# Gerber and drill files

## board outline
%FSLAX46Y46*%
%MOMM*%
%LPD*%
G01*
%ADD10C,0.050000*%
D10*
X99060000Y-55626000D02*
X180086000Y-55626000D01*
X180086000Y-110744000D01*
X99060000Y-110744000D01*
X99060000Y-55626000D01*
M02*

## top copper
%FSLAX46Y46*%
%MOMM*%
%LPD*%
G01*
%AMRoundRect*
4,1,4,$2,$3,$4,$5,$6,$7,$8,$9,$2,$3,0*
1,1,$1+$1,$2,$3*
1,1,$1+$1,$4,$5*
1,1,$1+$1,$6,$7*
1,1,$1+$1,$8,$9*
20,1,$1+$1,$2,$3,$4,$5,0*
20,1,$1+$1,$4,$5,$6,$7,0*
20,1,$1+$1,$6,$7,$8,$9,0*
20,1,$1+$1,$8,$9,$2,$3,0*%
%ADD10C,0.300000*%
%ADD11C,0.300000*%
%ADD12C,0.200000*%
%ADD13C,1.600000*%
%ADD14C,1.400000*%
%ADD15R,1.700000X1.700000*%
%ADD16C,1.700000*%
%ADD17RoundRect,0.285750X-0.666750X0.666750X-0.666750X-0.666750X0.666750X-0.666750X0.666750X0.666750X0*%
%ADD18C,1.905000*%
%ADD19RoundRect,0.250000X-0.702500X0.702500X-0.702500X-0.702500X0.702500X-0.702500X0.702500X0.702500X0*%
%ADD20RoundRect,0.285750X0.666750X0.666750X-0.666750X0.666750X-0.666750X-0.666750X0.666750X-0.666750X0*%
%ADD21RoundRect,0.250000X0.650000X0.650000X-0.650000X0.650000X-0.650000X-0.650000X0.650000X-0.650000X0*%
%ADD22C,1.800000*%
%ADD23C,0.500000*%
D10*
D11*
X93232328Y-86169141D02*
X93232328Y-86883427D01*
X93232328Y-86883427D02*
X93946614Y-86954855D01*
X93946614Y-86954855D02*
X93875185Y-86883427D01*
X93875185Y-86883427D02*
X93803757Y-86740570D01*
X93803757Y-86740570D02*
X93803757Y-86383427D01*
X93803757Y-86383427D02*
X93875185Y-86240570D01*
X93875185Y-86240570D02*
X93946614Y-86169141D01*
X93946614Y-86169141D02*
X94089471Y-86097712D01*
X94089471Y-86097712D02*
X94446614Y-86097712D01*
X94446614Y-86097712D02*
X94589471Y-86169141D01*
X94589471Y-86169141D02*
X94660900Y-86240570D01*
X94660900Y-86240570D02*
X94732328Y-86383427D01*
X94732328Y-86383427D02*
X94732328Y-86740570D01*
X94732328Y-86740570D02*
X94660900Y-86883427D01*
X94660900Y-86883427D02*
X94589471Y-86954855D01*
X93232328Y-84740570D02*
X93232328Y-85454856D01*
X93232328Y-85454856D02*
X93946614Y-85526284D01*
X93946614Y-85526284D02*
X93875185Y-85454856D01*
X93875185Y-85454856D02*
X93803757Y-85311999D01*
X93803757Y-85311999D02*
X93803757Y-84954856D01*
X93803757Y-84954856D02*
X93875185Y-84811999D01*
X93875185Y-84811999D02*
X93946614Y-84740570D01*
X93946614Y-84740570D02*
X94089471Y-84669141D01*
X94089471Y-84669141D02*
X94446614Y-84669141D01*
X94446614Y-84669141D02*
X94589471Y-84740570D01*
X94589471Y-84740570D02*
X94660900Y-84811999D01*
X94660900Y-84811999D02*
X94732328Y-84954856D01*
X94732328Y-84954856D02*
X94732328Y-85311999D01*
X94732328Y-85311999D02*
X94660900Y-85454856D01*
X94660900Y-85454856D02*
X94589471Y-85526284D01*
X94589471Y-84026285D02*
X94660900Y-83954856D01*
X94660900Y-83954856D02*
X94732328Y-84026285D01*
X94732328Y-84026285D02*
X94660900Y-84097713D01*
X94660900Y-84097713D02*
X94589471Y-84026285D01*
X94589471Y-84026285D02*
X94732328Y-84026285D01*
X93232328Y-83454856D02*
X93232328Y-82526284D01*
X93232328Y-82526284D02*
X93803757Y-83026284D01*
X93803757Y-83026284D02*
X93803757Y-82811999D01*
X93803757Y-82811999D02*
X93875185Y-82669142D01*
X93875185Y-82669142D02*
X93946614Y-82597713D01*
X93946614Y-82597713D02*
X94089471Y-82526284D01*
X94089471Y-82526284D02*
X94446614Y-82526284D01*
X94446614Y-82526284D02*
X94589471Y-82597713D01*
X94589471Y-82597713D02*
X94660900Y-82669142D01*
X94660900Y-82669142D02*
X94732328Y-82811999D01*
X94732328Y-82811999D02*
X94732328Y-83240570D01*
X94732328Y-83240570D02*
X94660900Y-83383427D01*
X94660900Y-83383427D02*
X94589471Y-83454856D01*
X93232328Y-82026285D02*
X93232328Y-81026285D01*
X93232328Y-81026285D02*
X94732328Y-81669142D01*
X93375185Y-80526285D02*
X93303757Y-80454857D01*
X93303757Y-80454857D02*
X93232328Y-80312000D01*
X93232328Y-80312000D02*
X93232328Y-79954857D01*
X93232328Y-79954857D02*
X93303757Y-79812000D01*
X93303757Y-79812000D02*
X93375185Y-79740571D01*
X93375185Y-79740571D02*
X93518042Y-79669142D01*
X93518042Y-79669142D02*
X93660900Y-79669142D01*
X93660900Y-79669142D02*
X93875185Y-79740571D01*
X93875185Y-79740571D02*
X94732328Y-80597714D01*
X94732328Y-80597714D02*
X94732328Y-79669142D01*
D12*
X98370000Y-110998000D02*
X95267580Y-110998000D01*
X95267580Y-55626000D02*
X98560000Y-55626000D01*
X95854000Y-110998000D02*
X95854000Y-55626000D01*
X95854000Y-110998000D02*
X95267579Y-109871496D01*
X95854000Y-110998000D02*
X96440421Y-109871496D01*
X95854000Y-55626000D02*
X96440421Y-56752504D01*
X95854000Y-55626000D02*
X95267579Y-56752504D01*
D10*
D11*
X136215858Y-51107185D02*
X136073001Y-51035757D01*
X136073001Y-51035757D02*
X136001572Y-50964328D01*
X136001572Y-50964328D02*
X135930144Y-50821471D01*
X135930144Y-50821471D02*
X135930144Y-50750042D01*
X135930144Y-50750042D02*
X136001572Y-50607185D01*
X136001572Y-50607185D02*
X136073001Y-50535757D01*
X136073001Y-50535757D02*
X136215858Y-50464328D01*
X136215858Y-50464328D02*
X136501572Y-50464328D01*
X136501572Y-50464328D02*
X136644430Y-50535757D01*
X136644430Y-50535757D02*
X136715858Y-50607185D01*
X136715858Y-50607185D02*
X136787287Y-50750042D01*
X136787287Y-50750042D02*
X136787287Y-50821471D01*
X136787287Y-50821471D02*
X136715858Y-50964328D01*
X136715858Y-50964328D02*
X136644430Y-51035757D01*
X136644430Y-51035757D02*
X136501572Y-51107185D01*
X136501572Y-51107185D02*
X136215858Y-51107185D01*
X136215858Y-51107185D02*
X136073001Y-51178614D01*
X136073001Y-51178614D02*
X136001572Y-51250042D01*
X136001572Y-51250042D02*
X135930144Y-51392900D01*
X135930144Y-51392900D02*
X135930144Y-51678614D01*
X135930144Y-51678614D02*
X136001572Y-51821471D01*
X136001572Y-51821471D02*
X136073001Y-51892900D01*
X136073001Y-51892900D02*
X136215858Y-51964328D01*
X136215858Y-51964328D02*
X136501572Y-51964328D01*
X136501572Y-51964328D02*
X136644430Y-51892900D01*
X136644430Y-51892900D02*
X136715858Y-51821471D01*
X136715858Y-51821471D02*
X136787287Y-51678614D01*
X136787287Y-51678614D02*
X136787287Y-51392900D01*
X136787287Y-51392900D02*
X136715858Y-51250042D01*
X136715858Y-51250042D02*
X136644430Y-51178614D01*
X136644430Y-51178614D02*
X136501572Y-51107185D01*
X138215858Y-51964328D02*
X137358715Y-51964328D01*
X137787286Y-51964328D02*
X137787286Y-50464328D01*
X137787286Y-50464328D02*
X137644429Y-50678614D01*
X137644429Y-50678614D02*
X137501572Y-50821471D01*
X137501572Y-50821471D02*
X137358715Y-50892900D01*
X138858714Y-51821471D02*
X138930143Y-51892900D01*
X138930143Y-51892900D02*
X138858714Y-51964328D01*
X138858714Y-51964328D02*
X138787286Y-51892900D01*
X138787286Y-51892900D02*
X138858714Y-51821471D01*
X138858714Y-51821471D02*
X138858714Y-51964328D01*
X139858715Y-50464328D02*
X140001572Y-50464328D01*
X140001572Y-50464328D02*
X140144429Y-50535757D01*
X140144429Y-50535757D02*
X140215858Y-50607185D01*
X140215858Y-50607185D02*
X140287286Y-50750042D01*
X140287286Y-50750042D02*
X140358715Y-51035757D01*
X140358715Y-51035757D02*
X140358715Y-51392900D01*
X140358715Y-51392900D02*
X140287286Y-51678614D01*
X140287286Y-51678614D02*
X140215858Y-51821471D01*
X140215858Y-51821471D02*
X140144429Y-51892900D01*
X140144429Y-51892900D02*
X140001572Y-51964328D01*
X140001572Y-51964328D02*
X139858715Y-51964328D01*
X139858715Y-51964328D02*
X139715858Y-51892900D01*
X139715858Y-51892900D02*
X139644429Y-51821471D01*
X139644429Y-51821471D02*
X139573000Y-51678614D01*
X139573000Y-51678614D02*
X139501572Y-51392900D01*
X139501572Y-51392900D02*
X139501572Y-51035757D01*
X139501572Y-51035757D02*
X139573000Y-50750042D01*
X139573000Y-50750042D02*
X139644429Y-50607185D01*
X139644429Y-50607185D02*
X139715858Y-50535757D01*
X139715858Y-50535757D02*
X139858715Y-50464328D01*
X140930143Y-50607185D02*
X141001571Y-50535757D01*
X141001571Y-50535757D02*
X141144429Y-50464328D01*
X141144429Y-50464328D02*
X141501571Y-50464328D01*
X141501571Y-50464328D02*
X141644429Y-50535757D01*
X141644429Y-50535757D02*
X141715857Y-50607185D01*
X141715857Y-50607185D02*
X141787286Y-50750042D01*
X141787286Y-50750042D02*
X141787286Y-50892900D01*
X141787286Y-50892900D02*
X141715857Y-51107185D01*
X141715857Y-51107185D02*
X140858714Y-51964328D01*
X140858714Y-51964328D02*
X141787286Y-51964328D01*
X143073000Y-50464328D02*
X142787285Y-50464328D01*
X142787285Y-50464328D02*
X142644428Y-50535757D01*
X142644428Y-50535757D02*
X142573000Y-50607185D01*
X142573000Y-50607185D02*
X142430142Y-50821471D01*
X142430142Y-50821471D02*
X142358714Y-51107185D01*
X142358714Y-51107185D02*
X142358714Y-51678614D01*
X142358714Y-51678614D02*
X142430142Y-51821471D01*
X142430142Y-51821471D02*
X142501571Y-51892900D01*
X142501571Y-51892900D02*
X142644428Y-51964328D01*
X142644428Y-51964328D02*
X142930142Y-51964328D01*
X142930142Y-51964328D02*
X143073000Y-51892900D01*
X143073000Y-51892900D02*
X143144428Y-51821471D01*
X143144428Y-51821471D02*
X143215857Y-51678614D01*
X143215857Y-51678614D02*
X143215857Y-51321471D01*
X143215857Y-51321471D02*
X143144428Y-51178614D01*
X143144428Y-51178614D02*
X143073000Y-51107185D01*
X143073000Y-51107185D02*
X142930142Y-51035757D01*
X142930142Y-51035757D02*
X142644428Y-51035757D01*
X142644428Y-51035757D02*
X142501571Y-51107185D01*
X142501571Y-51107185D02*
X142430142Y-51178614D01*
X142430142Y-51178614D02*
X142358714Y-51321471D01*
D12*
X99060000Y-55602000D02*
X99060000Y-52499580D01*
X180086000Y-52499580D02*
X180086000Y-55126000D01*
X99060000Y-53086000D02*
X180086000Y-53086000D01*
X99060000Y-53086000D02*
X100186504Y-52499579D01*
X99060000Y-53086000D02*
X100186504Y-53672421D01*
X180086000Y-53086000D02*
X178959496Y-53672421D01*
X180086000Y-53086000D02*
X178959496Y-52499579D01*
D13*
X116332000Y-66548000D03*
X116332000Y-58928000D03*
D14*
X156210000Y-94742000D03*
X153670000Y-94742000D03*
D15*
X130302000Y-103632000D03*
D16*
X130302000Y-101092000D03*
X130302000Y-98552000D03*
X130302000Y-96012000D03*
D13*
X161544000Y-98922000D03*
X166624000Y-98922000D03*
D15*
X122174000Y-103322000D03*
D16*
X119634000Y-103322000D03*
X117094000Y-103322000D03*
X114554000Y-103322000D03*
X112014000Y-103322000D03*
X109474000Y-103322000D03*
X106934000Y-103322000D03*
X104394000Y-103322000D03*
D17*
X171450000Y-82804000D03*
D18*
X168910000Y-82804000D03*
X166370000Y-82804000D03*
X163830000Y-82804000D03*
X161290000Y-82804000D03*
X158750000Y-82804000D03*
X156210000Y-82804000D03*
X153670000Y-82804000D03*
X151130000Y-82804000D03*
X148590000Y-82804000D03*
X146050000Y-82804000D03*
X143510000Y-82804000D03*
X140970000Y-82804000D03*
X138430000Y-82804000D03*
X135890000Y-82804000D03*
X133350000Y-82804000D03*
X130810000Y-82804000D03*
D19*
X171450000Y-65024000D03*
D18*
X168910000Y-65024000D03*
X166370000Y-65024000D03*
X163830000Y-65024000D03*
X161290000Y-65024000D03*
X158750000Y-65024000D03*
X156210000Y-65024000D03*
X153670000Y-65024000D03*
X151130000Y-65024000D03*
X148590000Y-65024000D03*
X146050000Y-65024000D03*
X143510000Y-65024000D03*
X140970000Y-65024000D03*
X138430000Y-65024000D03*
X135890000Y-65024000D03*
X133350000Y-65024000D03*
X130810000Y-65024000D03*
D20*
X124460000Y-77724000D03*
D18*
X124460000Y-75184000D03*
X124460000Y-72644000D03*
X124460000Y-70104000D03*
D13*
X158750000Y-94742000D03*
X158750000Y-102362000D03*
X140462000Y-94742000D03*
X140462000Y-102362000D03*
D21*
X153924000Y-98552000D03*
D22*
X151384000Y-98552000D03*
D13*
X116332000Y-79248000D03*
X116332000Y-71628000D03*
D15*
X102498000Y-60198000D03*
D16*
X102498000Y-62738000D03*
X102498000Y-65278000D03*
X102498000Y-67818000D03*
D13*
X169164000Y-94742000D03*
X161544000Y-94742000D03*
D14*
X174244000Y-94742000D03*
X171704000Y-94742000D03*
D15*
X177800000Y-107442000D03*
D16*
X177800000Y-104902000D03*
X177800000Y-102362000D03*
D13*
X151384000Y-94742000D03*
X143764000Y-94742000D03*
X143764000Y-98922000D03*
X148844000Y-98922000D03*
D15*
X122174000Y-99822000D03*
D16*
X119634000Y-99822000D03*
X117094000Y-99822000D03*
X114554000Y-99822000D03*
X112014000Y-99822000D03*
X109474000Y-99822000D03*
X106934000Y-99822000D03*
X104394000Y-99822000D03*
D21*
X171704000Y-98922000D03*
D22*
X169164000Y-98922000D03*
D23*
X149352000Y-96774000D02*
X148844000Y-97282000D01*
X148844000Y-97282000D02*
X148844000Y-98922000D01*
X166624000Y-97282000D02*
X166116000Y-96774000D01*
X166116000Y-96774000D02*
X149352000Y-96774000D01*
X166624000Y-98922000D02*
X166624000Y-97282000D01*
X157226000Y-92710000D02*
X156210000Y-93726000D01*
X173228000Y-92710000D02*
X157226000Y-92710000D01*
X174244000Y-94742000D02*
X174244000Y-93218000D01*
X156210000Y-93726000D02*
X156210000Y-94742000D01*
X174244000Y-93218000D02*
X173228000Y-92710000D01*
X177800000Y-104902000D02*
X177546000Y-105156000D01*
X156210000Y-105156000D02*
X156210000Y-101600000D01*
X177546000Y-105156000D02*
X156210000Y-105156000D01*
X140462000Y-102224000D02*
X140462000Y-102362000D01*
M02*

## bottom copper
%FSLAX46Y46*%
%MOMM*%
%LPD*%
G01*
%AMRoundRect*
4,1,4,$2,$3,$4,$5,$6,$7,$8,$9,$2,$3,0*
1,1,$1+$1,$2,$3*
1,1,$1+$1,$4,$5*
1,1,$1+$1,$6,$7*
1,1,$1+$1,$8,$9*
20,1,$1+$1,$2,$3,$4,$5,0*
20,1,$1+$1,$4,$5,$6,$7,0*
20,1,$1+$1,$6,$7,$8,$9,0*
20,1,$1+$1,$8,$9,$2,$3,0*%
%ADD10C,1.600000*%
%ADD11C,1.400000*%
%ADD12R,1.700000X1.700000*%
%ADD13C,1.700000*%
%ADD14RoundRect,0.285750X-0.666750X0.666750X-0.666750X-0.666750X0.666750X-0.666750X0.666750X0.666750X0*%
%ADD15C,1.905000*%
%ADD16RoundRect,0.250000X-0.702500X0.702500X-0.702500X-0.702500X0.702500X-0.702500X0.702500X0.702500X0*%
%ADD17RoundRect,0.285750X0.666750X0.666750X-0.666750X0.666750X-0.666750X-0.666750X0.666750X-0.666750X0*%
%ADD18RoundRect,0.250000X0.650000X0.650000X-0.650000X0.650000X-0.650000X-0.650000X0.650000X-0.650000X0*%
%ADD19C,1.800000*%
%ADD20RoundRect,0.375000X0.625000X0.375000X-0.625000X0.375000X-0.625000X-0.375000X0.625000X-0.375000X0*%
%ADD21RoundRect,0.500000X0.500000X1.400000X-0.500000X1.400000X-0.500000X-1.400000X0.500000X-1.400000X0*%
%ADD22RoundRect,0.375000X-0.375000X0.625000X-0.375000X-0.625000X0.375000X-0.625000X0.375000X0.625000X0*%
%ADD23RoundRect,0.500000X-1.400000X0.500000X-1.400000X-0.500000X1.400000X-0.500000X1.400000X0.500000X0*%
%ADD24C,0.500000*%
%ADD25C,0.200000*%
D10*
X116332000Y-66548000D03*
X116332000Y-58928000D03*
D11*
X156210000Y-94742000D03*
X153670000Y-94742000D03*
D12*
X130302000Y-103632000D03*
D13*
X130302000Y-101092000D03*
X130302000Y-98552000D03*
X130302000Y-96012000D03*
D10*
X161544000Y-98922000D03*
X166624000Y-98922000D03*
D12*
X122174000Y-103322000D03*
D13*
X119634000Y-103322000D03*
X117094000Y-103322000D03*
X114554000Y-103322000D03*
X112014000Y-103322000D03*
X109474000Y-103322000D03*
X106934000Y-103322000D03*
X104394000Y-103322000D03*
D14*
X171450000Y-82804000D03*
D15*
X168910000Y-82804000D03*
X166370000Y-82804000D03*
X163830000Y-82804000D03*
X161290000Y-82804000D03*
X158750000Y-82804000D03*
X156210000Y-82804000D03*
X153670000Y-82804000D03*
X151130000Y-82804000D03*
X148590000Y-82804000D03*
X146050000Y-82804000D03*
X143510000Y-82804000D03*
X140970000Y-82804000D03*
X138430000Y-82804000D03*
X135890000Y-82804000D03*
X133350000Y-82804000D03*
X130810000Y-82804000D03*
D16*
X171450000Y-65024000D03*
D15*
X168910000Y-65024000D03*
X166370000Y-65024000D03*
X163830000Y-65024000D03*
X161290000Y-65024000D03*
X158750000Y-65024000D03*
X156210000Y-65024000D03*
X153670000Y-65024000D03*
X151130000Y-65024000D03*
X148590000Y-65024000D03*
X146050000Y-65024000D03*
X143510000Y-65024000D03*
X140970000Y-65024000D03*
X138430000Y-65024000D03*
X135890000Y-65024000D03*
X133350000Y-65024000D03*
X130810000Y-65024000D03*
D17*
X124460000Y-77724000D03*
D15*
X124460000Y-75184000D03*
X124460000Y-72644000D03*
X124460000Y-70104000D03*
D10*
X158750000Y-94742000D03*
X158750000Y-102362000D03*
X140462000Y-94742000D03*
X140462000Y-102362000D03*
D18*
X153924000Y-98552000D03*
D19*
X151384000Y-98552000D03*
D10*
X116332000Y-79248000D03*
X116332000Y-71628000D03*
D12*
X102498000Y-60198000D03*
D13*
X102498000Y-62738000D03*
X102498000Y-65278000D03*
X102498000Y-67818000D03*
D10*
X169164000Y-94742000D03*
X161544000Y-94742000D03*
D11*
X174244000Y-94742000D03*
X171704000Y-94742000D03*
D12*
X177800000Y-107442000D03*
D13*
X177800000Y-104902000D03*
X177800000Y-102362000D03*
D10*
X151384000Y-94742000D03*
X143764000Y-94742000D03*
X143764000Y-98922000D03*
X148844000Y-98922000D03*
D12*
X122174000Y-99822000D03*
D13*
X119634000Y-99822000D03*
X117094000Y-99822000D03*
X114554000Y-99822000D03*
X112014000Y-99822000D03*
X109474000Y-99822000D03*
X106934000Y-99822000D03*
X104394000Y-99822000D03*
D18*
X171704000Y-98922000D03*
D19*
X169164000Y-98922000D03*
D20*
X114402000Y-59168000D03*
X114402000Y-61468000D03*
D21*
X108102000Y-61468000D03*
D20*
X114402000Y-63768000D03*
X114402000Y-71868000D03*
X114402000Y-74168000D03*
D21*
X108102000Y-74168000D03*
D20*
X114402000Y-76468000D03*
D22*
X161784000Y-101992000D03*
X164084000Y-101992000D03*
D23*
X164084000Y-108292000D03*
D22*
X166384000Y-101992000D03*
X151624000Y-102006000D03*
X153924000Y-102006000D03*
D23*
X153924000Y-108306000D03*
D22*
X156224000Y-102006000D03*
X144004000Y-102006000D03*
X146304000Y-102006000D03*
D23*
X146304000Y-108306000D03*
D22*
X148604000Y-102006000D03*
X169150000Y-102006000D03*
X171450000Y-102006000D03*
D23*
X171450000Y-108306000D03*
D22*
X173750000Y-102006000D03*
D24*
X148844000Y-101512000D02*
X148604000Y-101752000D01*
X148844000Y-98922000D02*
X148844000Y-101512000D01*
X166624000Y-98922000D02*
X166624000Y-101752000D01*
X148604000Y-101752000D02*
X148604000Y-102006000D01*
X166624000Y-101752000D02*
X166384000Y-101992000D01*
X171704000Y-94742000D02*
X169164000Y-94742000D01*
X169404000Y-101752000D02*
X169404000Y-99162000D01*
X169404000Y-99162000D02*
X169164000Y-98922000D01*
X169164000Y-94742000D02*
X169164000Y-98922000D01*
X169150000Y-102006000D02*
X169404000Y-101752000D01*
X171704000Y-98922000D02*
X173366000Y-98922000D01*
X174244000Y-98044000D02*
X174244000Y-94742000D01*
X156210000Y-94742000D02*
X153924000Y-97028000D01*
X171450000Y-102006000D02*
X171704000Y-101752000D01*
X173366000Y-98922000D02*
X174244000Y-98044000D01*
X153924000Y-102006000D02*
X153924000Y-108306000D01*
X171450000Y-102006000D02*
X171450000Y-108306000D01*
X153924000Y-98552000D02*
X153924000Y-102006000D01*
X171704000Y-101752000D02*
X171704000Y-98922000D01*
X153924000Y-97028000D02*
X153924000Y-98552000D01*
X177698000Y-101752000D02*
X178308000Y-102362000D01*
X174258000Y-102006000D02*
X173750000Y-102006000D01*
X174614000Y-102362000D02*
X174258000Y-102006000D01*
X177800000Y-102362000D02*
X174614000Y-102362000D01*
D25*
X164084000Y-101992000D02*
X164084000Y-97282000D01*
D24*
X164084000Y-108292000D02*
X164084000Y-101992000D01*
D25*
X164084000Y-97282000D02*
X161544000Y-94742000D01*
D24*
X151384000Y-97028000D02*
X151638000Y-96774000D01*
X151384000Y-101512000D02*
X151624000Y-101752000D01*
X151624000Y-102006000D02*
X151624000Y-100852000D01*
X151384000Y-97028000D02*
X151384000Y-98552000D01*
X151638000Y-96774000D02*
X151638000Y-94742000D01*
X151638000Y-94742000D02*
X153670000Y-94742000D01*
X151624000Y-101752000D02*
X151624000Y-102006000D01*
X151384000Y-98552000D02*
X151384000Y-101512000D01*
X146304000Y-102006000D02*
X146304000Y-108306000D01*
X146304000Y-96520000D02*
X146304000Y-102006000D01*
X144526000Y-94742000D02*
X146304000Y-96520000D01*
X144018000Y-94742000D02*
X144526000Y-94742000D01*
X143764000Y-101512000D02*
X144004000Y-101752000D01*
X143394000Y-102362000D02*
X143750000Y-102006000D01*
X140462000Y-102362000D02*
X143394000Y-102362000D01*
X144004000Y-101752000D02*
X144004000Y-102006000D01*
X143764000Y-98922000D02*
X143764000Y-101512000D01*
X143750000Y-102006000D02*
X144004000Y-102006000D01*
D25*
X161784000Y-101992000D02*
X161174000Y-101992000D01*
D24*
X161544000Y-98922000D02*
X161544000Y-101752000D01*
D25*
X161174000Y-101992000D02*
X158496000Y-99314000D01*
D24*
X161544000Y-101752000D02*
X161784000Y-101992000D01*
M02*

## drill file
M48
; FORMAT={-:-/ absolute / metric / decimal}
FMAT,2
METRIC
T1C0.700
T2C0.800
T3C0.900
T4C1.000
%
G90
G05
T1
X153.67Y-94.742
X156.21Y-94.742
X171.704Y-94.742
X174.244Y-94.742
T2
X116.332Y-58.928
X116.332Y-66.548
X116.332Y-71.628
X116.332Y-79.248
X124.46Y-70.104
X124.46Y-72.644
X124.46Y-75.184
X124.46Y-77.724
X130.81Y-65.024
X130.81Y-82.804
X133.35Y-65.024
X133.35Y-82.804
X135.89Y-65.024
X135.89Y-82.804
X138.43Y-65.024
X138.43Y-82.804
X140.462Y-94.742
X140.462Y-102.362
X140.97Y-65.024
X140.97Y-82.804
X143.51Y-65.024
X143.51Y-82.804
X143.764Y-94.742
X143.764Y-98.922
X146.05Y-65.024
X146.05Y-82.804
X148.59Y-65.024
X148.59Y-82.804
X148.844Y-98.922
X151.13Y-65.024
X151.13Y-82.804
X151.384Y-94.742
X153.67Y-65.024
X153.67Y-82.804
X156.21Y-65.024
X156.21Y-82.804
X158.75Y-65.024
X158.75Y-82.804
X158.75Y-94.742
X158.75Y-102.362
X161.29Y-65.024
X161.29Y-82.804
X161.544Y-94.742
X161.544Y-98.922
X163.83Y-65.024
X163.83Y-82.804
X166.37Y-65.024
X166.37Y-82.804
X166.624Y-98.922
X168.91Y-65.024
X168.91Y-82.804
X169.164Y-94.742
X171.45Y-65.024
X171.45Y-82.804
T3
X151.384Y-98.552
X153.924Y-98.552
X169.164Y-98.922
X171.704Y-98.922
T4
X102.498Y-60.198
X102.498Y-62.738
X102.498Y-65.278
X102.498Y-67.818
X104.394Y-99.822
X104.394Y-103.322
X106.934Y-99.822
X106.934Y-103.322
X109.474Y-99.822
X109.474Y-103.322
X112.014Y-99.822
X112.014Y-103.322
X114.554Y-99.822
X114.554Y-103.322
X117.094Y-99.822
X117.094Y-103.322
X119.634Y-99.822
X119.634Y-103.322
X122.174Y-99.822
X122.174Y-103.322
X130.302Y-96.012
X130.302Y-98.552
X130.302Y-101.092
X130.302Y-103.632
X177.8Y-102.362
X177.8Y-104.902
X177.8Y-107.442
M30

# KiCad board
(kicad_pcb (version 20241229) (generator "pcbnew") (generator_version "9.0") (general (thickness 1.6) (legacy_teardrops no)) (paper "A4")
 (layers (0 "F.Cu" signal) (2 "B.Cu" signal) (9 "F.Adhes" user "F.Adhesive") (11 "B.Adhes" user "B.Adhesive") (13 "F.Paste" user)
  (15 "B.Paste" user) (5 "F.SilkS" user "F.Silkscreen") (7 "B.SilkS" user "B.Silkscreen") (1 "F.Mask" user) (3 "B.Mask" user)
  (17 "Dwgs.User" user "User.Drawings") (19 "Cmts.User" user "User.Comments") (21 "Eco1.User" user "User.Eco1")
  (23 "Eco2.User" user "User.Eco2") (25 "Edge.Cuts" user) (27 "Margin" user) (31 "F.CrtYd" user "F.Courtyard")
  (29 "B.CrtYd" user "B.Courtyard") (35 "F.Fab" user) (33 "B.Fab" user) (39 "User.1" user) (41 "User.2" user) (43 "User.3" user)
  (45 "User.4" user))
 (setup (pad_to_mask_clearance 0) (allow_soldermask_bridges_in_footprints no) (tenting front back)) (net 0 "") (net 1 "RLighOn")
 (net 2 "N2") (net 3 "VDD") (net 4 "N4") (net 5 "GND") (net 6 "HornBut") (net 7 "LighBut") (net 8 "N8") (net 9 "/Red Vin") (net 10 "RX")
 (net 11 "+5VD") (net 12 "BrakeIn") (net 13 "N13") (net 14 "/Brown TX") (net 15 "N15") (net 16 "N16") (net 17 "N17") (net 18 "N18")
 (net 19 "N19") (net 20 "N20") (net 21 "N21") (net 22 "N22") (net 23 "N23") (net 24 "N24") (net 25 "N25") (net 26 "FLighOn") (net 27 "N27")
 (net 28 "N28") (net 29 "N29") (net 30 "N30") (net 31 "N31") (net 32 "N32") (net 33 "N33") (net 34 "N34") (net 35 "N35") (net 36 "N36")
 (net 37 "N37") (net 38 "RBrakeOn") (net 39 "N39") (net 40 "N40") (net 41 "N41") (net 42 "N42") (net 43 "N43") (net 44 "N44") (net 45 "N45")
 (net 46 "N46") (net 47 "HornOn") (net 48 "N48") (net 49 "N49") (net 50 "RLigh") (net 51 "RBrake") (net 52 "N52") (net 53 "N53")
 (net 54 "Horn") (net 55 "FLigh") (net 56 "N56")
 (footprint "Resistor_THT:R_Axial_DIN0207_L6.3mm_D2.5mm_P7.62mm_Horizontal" (layer "F.Cu") (at 116.332 66.548 90)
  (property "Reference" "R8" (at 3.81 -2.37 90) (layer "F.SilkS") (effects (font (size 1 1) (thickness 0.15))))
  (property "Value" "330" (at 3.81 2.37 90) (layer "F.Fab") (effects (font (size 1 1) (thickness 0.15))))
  (pad "1" thru_hole circle (at 0 0 90) (size 1.6 1.6) (drill 0.8) (layers "*.Cu" "*.Mask") (remove_unused_layers no) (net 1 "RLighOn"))
  (pad "2" thru_hole circle (at 7.62 0 90) (size 1.6 1.6) (drill 0.8) (layers "*.Cu" "*.Mask") (remove_unused_layers no) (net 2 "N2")))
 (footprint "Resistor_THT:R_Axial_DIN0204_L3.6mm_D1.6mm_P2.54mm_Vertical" (layer "F.Cu") (at 156.21 94.742 180)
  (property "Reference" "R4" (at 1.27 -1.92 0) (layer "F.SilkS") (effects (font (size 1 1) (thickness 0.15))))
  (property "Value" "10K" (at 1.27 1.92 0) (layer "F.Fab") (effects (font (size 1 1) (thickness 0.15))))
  (pad "1" thru_hole circle (at 0 0 180) (size 1.4 1.4) (drill 0.7) (layers "*.Cu" "*.Mask") (remove_unused_layers no) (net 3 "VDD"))
  (pad "2" thru_hole circle (at 2.54 0 180) (size 1.4 1.4) (drill 0.7) (layers "*.Cu" "*.Mask") (remove_unused_layers no) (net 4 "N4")))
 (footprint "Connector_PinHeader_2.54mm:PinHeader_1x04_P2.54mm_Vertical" (layer "F.Cu") (at 130.302 103.632 180)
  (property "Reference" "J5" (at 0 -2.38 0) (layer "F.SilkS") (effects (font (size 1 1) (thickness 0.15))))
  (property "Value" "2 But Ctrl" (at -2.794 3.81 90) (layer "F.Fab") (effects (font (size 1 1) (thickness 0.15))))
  (pad "1" thru_hole rect (at 0 0 180) (size 1.7 1.7) (drill 1) (layers "*.Cu" "*.Mask") (remove_unused_layers no) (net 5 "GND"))
  (pad "2" thru_hole circle (at 0 2.54 180) (size 1.7 1.7) (drill 1) (layers "*.Cu" "*.Mask") (remove_unused_layers no) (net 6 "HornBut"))
  (pad "3" thru_hole circle (at 0 5.08 180) (size 1.7 1.7) (drill 1) (layers "*.Cu" "*.Mask") (remove_unused_layers no) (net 5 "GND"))
  (pad "4" thru_hole circle (at 0 7.62 180) (size 1.7 1.7) (drill 1) (layers "*.Cu" "*.Mask") (remove_unused_layers no) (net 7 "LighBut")))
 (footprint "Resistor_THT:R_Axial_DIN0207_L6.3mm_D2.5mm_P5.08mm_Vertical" (layer "F.Cu") (at 161.544 98.922)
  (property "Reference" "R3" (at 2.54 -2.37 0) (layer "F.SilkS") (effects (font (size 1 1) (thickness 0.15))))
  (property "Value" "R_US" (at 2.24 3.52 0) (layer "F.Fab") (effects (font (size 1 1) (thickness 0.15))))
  (pad "1" thru_hole circle (at 0 0) (size 1.6 1.6) (drill 0.8) (layers "*.Cu" "*.Mask") (remove_unused_layers no) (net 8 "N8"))
  (pad "2" thru_hole circle (at 5.08 0) (size 1.6 1.6) (drill 0.8) (layers "*.Cu" "*.Mask") (remove_unused_layers no) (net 5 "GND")))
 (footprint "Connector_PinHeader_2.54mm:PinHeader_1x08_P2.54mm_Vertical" (layer "F.Cu") (at 122.174 103.322 -90)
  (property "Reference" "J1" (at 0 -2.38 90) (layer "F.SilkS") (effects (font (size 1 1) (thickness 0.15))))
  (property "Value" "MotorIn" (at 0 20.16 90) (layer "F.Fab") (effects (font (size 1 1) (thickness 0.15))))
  (pad "1" thru_hole rect (at 0 0 270) (size 1.7 1.7) (drill 1) (layers "*.Cu" "*.Mask") (remove_unused_layers no) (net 5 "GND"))
  (pad "2" thru_hole circle (at 0 2.54 270) (size 1.7 1.7) (drill 1) (layers "*.Cu" "*.Mask") (remove_unused_layers no) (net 3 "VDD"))
  (pad "3" thru_hole circle (at 0 5.08 270) (size 1.7 1.7) (drill 1) (layers "*.Cu" "*.Mask") (remove_unused_layers no) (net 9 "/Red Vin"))
  (pad "4" thru_hole circle (at 0 7.62 270) (size 1.7 1.7) (drill 1) (layers "*.Cu" "*.Mask") (remove_unused_layers no) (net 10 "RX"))
  (pad "5" thru_hole circle (at 0 10.16 270) (size 1.7 1.7) (drill 1) (layers "*.Cu" "*.Mask") (remove_unused_layers no) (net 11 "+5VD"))
  (pad "6" thru_hole circle (at 0 12.7 270) (size 1.7 1.7) (drill 1) (layers "*.Cu" "*.Mask") (remove_unused_layers no) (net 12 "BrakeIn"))
  (pad "7" thru_hole circle (at 0 15.24 270) (size 1.7 1.7) (drill 1) (layers "*.Cu" "*.Mask") (remove_unused_layers no) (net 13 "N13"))
  (pad "8" thru_hole circle (at 0 17.78 270) (size 1.7 1.7) (drill 1) (layers "*.Cu" "*.Mask") (remove_unused_layers no)
   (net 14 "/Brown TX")))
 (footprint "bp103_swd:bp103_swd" (layer "F.Cu") (at 156.21 73.914 -90)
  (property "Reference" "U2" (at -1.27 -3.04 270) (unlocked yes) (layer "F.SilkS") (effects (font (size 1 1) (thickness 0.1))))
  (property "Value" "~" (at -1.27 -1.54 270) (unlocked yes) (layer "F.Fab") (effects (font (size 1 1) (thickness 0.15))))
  (pad "1" thru_hole roundrect (at 8.89 -15.24 270) (size 1.905 1.905) (drill 0.8) (layers "*.Cu" "*.Mask") (remove_unused_layers no)
   (roundrect_rratio 0.15) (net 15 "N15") (thermal_bridge_angle 45))
  (pad "2" thru_hole circle (at 8.89 -12.7 270) (size 1.905 1.905) (drill 0.8) (layers "*.Cu" "*.Mask") (remove_unused_layers no)
   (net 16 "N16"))
  (pad "3" thru_hole circle (at 8.89 -10.16 270) (size 1.905 1.905) (drill 0.8) (layers "*.Cu" "*.Mask") (remove_unused_layers no)
   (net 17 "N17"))
  (pad "4" thru_hole circle (at 8.89 -7.62 270) (size 1.905 1.905) (drill 0.8) (layers "*.Cu" "*.Mask") (remove_unused_layers no)
   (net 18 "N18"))
  (pad "5" thru_hole circle (at 8.89 -5.08 270) (size 1.905 1.905) (drill 0.8) (layers "*.Cu" "*.Mask") (remove_unused_layers no)
   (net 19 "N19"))
  (pad "6" thru_hole circle (at 8.89 -2.54 270) (size 1.905 1.905) (drill 0.8) (layers "*.Cu" "*.Mask") (remove_unused_layers no)
   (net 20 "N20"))
  (pad "7" thru_hole circle (at 8.89 0 270) (size 1.905 1.905) (drill 0.8) (layers "*.Cu" "*.Mask") (remove_unused_layers no) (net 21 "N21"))
  (pad "8" thru_hole circle (at 8.89 2.54 270) (size 1.905 1.905) (drill 0.8) (layers "*.Cu" "*.Mask") (remove_unused_layers no)
   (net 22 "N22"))
  (pad "9" thru_hole circle (at 8.89 5.08 270) (size 1.905 1.905) (drill 0.8) (layers "*.Cu" "*.Mask") (remove_unused_layers no)
   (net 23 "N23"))
  (pad "10" thru_hole circle (at 8.89 7.62 270) (size 1.905 1.905) (drill 0.8) (layers "*.Cu" "*.Mask") (remove_unused_layers no)
   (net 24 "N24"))
  (pad "11" thru_hole circle (at 8.89 10.16 270) (size 1.905 1.905) (drill 0.8) (layers "*.Cu" "*.Mask") (remove_unused_layers no)
   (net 10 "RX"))
  (pad "12" thru_hole circle (at 8.89 12.7 270) (size 1.905 1.905) (drill 0.8) (layers "*.Cu" "*.Mask") (remove_unused_layers no)
   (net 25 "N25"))
  (pad "13" thru_hole circle (at 8.89 15.24 270) (size 1.905 1.905) (drill 0.8) (layers "*.Cu" "*.Mask") (remove_unused_layers no)
   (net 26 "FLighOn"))
  (pad "14" thru_hole circle (at 8.89 17.78 270) (size 1.905 1.905) (drill 0.8) (layers "*.Cu" "*.Mask") (remove_unused_layers no)
   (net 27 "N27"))
  (pad "15" thru_hole circle (at 8.89 20.32 270) (size 1.905 1.905) (drill 0.8) (layers "*.Cu" "*.Mask") (remove_unused_layers no)
   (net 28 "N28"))
  (pad "16" thru_hole circle (at 8.89 22.86 270) (size 1.905 1.905) (drill 0.8) (layers "*.Cu" "*.Mask") (remove_unused_layers no)
   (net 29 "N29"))
  (pad "17" thru_hole circle (at 8.89 25.4 270) (size 1.905 1.905) (drill 0.8) (layers "*.Cu" "*.Mask") (remove_unused_layers no)
   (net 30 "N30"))
  (pad "18" thru_hole roundrect (at -8.89 -15.24 270) (size 1.905 1.905) (drill 0.8) (layers "*.Cu" "*.Mask") (remove_unused_layers no)
   (roundrect_rratio 0.1312335958) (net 5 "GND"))
  (pad "19" thru_hole circle (at -8.89 -12.7 270) (size 1.905 1.905) (drill 0.8) (layers "*.Cu" "*.Mask") (remove_unused_layers no)
   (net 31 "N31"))
  (pad "20" thru_hole circle (at -8.89 -10.16 270) (size 1.905 1.905) (drill 0.8) (layers "*.Cu" "*.Mask") (remove_unused_layers no)
   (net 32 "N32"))
  (pad "21" thru_hole circle (at -8.89 -7.62 270) (size 1.905 1.905) (drill 0.8) (layers "*.Cu" "*.Mask") (remove_unused_layers no)
   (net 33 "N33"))
  (pad "22" thru_hole circle (at -8.89 -5.08 270) (size 1.905 1.905) (drill 0.8) (layers "*.Cu" "*.Mask") (remove_unused_layers no)
   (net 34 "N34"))
  (pad "23" thru_hole circle (at -8.89 -2.54 270) (size 1.905 1.905) (drill 0.8) (layers "*.Cu" "*.Mask") (remove_unused_layers no)
   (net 12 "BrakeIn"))
  (pad "24" thru_hole circle (at -8.89 0 270) (size 1.905 1.905) (drill 0.8) (layers "*.Cu" "*.Mask") (remove_unused_layers no)
   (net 7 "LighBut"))
  (pad "25" thru_hole circle (at -8.89 2.54 270) (size 1.905 1.905) (drill 0.8) (layers "*.Cu" "*.Mask") (remove_unused_layers no)
   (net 6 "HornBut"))
  (pad "26" thru_hole circle (at -8.89 5.08 270) (size 1.905 1.905) (drill 0.8) (layers "*.Cu" "*.Mask") (remove_unused_layers no)
   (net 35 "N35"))
  (pad "27" thru_hole circle (at -8.89 7.62 270) (size 1.905 1.905) (drill 0.8) (layers "*.Cu" "*.Mask") (remove_unused_layers no)
   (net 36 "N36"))
  (pad "28" thru_hole circle (at -8.89 10.16 270) (size 1.905 1.905) (drill 0.8) (layers "*.Cu" "*.Mask") (remove_unused_layers no)
   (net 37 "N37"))
  (pad "29" thru_hole circle (at -8.89 12.7 270) (size 1.905 1.905) (drill 0.8) (layers "*.Cu" "*.Mask") (remove_unused_layers no)
   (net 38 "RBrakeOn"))
  (pad "30" thru_hole circle (at -8.89 15.24 270) (size 1.905 1.905) (drill 0.8) (layers "*.Cu" "*.Mask") (remove_unused_layers no)
   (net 1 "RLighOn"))
  (pad "31" thru_hole circle (at -8.89 17.78 270) (size 1.905 1.905) (drill 0.8) (layers "*.Cu" "*.Mask") (remove_unused_layers no)
   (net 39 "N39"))
  (pad "32" thru_hole circle (at -8.89 20.32 270) (size 1.905 1.905) (drill 0.8) (layers "*.Cu" "*.Mask") (remove_unused_layers no)
   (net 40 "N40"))
  (pad "33" thru_hole circle (at -8.89 22.86 270) (size 1.905 1.905) (drill 0.8) (layers "*.Cu" "*.Mask") (remove_unused_layers no)
   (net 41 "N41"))
  (pad "34" thru_hole circle (at -8.89 25.4 270) (size 1.905 1.905) (drill 0.8) (layers "*.Cu" "*.Mask") (remove_unused_layers no)
   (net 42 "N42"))
  (pad "35" thru_hole roundrect (at 3.81 31.75 180) (size 1.905 1.905) (drill 0.8) (layers "*.Cu" "*.Mask") (remove_unused_layers no)
   (roundrect_rratio 0.15) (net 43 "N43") (thermal_bridge_angle 45))
  (pad "36" thru_hole circle (at 1.27 31.75 180) (size 1.905 1.905) (drill 0.8) (layers "*.Cu" "*.Mask") (remove_unused_layers no)
   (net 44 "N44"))
  (pad "37" thru_hole circle (at -1.27 31.75 180) (size 1.905 1.905) (drill 0.8) (layers "*.Cu" "*.Mask") (remove_unused_layers no)
   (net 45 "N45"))
  (pad "38" thru_hole circle (at -3.81 31.75 180) (size 1.905 1.905) (drill 0.8) (layers "*.Cu" "*.Mask") (remove_unused_layers no)
   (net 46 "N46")))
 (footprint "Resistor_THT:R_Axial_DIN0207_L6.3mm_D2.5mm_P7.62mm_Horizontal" (layer "F.Cu") (at 158.75 94.742 -90)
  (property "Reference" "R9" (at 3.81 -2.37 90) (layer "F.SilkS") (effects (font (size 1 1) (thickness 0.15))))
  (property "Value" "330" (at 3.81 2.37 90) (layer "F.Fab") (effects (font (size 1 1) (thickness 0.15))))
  (pad "1" thru_hole circle (at 0 0 270) (size 1.6 1.6) (drill 0.8) (layers "*.Cu" "*.Mask") (remove_unused_layers no) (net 26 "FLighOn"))
  (pad "2" thru_hole circle (at 7.62 0 270) (size 1.6 1.6) (drill 0.8) (layers "*.Cu" "*.Mask") (remove_unused_layers no) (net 8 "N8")))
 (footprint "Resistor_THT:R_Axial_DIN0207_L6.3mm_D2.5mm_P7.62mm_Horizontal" (layer "F.Cu") (at 140.462 94.742 -90)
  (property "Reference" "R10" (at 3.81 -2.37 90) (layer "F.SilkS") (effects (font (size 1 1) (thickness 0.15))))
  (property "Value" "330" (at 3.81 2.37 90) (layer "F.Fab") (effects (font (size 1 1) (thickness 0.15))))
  (pad "1" thru_hole circle (at 0 0 270) (size 1.6 1.6) (drill 0.8) (layers "*.Cu" "*.Mask") (remove_unused_layers no) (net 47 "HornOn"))
  (pad "2" thru_hole circle (at 7.62 0 270) (size 1.6 1.6) (drill 0.8) (layers "*.Cu" "*.Mask") (remove_unused_layers no) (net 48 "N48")))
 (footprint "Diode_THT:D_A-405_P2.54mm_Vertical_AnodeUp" (layer "F.Cu") (at 153.924 98.552 180)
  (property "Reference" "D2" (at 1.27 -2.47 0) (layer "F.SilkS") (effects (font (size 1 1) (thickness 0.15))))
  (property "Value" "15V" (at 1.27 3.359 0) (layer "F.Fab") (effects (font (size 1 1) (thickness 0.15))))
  (pad "1" thru_hole roundrect (at 0 0 180) (size 1.8 1.8) (drill 0.9) (layers "*.Cu" "*.Mask") (remove_unused_layers no)
   (roundrect_rratio 0.138889) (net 3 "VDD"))
  (pad "2" thru_hole circle (at 2.54 0 180) (size 1.8 1.8) (drill 0.9) (layers "*.Cu" "*.Mask") (remove_unused_layers no) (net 4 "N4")))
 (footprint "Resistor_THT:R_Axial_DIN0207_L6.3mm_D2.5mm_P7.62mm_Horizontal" (layer "F.Cu") (at 116.332 79.248 90)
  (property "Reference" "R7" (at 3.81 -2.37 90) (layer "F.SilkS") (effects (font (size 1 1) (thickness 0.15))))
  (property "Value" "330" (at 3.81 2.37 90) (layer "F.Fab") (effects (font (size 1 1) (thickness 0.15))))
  (pad "1" thru_hole circle (at 0 0 90) (size 1.6 1.6) (drill 0.8) (layers "*.Cu" "*.Mask") (remove_unused_layers no) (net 38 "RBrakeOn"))
  (pad "2" thru_hole circle (at 7.62 0 90) (size 1.6 1.6) (drill 0.8) (layers "*.Cu" "*.Mask") (remove_unused_layers no) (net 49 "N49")))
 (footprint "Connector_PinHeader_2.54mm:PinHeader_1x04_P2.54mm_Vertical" (layer "F.Cu") (at 102.498 60.198)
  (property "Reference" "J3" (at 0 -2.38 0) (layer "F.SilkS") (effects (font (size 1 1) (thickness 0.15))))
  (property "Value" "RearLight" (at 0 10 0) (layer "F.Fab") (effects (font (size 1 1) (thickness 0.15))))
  (pad "1" thru_hole rect (at 0 0) (size 1.7 1.7) (drill 1) (layers "*.Cu" "*.Mask") (remove_unused_layers no) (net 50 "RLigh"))
  (pad "2" thru_hole circle (at 0 2.54) (size 1.7 1.7) (drill 1) (layers "*.Cu" "*.Mask") (remove_unused_layers no) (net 3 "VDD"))
  (pad "3" thru_hole circle (at 0 5.08) (size 1.7 1.7) (drill 1) (layers "*.Cu" "*.Mask") (remove_unused_layers no) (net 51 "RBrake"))
  (pad "4" thru_hole circle (at 0 7.62) (size 1.7 1.7) (drill 1) (layers "*.Cu" "*.Mask") (remove_unused_layers no) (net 3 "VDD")))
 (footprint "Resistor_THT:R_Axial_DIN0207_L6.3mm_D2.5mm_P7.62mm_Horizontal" (layer "F.Cu") (at 169.164 94.742 180)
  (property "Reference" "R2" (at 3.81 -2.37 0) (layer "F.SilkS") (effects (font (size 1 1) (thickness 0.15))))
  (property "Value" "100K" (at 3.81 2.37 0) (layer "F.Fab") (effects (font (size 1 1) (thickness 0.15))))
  (pad "1" thru_hole circle (at 0 0 180) (size 1.6 1.6) (drill 0.8) (layers "*.Cu" "*.Mask") (remove_unused_layers no) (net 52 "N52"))
  (pad "2" thru_hole circle (at 7.62 0 180) (size 1.6 1.6) (drill 0.8) (layers "*.Cu" "*.Mask") (remove_unused_layers no) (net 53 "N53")))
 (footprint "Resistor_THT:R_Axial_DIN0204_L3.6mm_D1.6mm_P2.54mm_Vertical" (layer "F.Cu") (at 174.244 94.742 180)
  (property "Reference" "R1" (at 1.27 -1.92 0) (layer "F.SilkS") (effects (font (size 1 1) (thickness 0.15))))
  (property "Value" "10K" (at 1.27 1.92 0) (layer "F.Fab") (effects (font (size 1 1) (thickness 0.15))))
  (pad "1" thru_hole circle (at 0 0 180) (size 1.4 1.4) (drill 0.7) (layers "*.Cu" "*.Mask") (remove_unused_layers no) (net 3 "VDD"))
  (pad "2" thru_hole circle (at 2.54 0 180) (size 1.4 1.4) (drill 0.7) (layers "*.Cu" "*.Mask") (remove_unused_layers no) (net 52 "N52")))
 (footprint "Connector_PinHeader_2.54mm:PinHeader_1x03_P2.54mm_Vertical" (layer "F.Cu") (at 177.8 107.442 180)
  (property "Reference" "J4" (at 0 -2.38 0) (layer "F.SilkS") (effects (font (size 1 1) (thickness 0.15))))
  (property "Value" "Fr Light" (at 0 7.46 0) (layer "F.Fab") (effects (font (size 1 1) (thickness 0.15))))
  (pad "1" thru_hole rect (at 0 0 180) (size 1.7 1.7) (drill 1) (layers "*.Cu" "*.Mask") (remove_unused_layers no) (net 5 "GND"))
  (pad "2" thru_hole circle (at 0 2.54 180) (size 1.7 1.7) (drill 1) (layers "*.Cu" "*.Mask") (remove_unused_layers no) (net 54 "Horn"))
  (pad "3" thru_hole circle (at 0 5.08 180) (size 1.7 1.7) (drill 1) (layers "*.Cu" "*.Mask") (remove_unused_layers no) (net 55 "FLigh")))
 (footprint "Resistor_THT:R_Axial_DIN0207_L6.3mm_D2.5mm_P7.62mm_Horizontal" (layer "F.Cu") (at 151.384 94.742 180)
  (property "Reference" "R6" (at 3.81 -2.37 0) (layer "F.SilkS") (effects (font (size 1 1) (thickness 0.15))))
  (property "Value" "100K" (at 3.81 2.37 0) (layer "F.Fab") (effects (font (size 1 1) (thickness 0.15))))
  (pad "1" thru_hole circle (at 0 0 180) (size 1.6 1.6) (drill 0.8) (layers "*.Cu" "*.Mask") (remove_unused_layers no) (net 4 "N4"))
  (pad "2" thru_hole circle (at 7.62 0 180) (size 1.6 1.6) (drill 0.8) (layers "*.Cu" "*.Mask") (remove_unused_layers no) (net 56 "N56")))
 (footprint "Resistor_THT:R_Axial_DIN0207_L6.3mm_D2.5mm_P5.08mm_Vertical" (layer "F.Cu") (at 143.764 98.922)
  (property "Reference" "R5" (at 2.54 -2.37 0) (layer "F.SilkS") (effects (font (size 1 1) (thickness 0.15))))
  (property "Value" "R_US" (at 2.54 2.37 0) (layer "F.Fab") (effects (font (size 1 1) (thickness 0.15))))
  (pad "1" thru_hole circle (at 0 0) (size 1.6 1.6) (drill 0.8) (layers "*.Cu" "*.Mask") (remove_unused_layers no) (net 48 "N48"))
  (pad "2" thru_hole circle (at 5.08 0) (size 1.6 1.6) (drill 0.8) (layers "*.Cu" "*.Mask") (remove_unused_layers no) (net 5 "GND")))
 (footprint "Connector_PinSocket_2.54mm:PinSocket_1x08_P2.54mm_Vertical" (layer "F.Cu") (at 122.174 99.822 -90)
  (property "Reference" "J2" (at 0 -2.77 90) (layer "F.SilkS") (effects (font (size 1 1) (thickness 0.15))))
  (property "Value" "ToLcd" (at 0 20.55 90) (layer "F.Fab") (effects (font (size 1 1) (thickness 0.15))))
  (pad "1" thru_hole rect (at 0 0 270) (size 1.7 1.7) (drill 1) (layers "*.Cu" "*.Mask") (remove_unused_layers no) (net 5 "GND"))
  (pad "2" thru_hole circle (at 0 2.54 270) (size 1.7 1.7) (drill 1) (layers "*.Cu" "*.Mask") (remove_unused_layers no) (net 3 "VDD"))
  (pad "3" thru_hole circle (at 0 5.08 270) (size 1.7 1.7) (drill 1) (layers "*.Cu" "*.Mask") (remove_unused_layers no) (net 9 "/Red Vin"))
  (pad "4" thru_hole circle (at 0 7.62 270) (size 1.7 1.7) (drill 1) (layers "*.Cu" "*.Mask") (remove_unused_layers no) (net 10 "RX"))
  (pad "5" thru_hole circle (at 0 10.16 270) (size 1.7 1.7) (drill 1) (layers "*.Cu" "*.Mask") (remove_unused_layers no) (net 11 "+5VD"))
  (pad "6" thru_hole circle (at 0 12.7 270) (size 1.7 1.7) (drill 1) (layers "*.Cu" "*.Mask") (remove_unused_layers no) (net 12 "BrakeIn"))
  (pad "7" thru_hole circle (at 0 15.24 270) (size 1.7 1.7) (drill 1) (layers "*.Cu" "*.Mask") (remove_unused_layers no) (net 13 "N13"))
  (pad "8" thru_hole circle (at 0 17.78 270) (size 1.7 1.7) (drill 1) (layers "*.Cu" "*.Mask") (remove_unused_layers no)
   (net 14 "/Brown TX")))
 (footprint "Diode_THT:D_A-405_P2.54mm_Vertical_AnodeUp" (layer "F.Cu") (at 171.704 98.922 180)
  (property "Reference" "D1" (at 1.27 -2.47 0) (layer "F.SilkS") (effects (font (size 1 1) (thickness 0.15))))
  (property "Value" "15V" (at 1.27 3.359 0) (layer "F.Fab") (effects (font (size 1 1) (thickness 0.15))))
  (pad "1" thru_hole roundrect (at 0 0 180) (size 1.8 1.8) (drill 0.9) (layers "*.Cu" "*.Mask") (remove_unused_layers no)
   (roundrect_rratio 0.138889) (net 3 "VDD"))
  (pad "2" thru_hole circle (at 2.54 0 180) (size 1.8 1.8) (drill 0.9) (layers "*.Cu" "*.Mask") (remove_unused_layers no) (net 52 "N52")))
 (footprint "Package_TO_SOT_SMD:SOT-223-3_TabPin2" (layer "B.Cu") (at 111.252 61.468 180)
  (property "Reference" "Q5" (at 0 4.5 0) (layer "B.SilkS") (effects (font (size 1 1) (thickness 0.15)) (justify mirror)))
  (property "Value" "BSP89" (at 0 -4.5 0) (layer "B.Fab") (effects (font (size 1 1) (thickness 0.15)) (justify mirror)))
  (pad "1" smd roundrect (at -3.15 2.3 180) (size 2 1.5) (layers "B.Cu" "B.Mask" "B.Paste") (roundrect_rratio 0.25) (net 2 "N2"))
  (pad "2" smd roundrect (at -3.15 0 180) (size 2 1.5) (layers "B.Cu" "B.Mask" "B.Paste") (roundrect_rratio 0.25) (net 50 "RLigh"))
  (pad "2" smd roundrect (at 3.15 0 180) (size 2 3.8) (layers "B.Cu" "B.Mask" "B.Paste") (roundrect_rratio 0.25) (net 50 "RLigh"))
  (pad "3" smd roundrect (at -3.15 -2.3 180) (size 2 1.5) (layers "B.Cu" "B.Mask" "B.Paste") (roundrect_rratio 0.25) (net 5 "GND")))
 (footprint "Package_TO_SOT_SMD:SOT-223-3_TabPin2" (layer "B.Cu") (at 111.252 74.168 180)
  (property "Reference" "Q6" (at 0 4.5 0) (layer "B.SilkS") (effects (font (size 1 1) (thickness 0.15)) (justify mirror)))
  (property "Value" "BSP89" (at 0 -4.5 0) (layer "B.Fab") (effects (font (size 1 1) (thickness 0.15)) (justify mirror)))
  (pad "1" smd roundrect (at -3.15 2.3 180) (size 2 1.5) (layers "B.Cu" "B.Mask" "B.Paste") (roundrect_rratio 0.25) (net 49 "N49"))
  (pad "2" smd roundrect (at -3.15 0 180) (size 2 1.5) (layers "B.Cu" "B.Mask" "B.Paste") (roundrect_rratio 0.25) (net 51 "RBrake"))
  (pad "2" smd roundrect (at 3.15 0 180) (size 2 3.8) (layers "B.Cu" "B.Mask" "B.Paste") (roundrect_rratio 0.25) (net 51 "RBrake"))
  (pad "3" smd roundrect (at -3.15 -2.3 180) (size 2 1.5) (layers "B.Cu" "B.Mask" "B.Paste") (roundrect_rratio 0.25) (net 5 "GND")))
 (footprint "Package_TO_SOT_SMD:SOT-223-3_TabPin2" (layer "B.Cu") (at 164.084 105.142 -90)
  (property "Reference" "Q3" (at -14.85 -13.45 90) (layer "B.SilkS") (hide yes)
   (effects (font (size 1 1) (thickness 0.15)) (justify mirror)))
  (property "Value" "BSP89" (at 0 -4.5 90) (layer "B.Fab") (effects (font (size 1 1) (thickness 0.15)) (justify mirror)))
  (pad "1" smd roundrect (at -3.15 2.3 270) (size 2 1.5) (layers "B.Cu" "B.Mask" "B.Paste") (roundrect_rratio 0.25) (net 8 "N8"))
  (pad "2" smd roundrect (at -3.15 0 270) (size 2 1.5) (layers "B.Cu" "B.Mask" "B.Paste") (roundrect_rratio 0.25) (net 53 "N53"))
  (pad "2" smd roundrect (at 3.15 0 270) (size 2 3.8) (layers "B.Cu" "B.Mask" "B.Paste") (roundrect_rratio 0.25) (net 53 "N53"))
  (pad "3" smd roundrect (at -3.15 -2.3 270) (size 2 1.5) (layers "B.Cu" "B.Mask" "B.Paste") (roundrect_rratio 0.25) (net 5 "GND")))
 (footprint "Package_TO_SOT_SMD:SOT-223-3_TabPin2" (layer "B.Cu") (at 153.924 105.156 -90)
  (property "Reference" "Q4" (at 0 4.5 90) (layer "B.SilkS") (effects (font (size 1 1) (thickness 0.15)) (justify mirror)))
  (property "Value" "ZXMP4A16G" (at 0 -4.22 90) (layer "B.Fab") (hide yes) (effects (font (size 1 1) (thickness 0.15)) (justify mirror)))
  (pad "1" smd roundrect (at -3.15 2.3 270) (size 2 1.5) (layers "B.Cu" "B.Mask" "B.Paste") (roundrect_rratio 0.25) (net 4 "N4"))
  (pad "2" smd roundrect (at -3.15 0 270) (size 2 1.5) (layers "B.Cu" "B.Mask" "B.Paste") (roundrect_rratio 0.25) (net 3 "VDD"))
  (pad "2" smd roundrect (at 3.15 0 270) (size 2 3.8) (layers "B.Cu" "B.Mask" "B.Paste") (roundrect_rratio 0.25) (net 3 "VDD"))
  (pad "3" smd roundrect (at -3.15 -2.3 270) (size 2 1.5) (layers "B.Cu" "B.Mask" "B.Paste") (roundrect_rratio 0.25) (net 54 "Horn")))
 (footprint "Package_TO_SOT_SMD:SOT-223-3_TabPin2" (layer "B.Cu") (at 146.304 105.156 -90)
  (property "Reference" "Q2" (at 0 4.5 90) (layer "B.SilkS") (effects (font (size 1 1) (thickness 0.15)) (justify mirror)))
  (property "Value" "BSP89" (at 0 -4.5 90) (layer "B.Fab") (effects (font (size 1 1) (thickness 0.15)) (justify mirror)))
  (pad "1" smd roundrect (at -3.15 2.3 270) (size 2 1.5) (layers "B.Cu" "B.Mask" "B.Paste") (roundrect_rratio 0.25) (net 48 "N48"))
  (pad "2" smd roundrect (at -3.15 0 270) (size 2 1.5) (layers "B.Cu" "B.Mask" "B.Paste") (roundrect_rratio 0.25) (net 56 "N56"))
  (pad "2" smd roundrect (at 3.15 0 270) (size 2 3.8) (layers "B.Cu" "B.Mask" "B.Paste") (roundrect_rratio 0.25) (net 56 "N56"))
  (pad "3" smd roundrect (at -3.15 -2.3 270) (size 2 1.5) (layers "B.Cu" "B.Mask" "B.Paste") (roundrect_rratio 0.25) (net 5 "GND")))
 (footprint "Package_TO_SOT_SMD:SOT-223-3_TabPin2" (layer "B.Cu") (at 171.45 105.156 -90)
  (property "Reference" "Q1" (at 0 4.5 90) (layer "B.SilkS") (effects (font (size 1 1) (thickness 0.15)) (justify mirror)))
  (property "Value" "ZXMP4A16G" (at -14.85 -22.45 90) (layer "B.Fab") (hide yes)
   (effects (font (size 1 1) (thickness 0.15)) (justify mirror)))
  (pad "1" smd roundrect (at -3.15 2.3 270) (size 2 1.5) (layers "B.Cu" "B.Mask" "B.Paste") (roundrect_rratio 0.25) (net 52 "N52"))
  (pad "2" smd roundrect (at -3.15 0 270) (size 2 1.5) (layers "B.Cu" "B.Mask" "B.Paste") (roundrect_rratio 0.25) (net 3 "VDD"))
  (pad "2" smd roundrect (at 3.15 0 270) (size 2 3.8) (layers "B.Cu" "B.Mask" "B.Paste") (roundrect_rratio 0.25) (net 3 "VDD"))
  (pad "3" smd roundrect (at -3.15 -2.3 270) (size 2 1.5) (layers "B.Cu" "B.Mask" "B.Paste") (roundrect_rratio 0.25) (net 55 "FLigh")))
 (gr_rect (start 99.06 55.626) (end 180.086 110.744) (stroke (width 0.05) (type default)) (fill no) (layer "Edge.Cuts"))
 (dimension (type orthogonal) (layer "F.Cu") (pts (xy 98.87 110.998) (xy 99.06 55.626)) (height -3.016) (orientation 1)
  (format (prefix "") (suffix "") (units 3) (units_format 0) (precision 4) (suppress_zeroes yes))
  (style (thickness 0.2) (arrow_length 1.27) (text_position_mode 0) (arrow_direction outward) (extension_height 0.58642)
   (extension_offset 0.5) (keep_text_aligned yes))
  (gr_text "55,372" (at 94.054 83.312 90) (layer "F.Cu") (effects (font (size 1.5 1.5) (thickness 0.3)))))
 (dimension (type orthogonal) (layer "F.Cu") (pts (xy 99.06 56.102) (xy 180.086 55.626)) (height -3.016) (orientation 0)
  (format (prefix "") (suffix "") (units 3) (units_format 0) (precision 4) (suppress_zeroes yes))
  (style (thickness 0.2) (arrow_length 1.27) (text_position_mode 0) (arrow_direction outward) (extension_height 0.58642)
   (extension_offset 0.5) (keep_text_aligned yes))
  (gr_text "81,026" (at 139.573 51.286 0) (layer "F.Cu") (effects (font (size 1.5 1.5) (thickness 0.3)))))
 (segment (start 149.352 96.774) (end 148.844 97.282) (width 0.5) (layer "F.Cu") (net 5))
 (segment (start 148.844 97.282) (end 148.844 98.922) (width 0.5) (layer "F.Cu") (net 5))
 (segment (start 166.624 97.282) (end 166.116 96.774) (width 0.5) (layer "F.Cu") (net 5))
 (segment (start 166.116 96.774) (end 149.352 96.774) (width 0.5) (layer "F.Cu") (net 5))
 (segment (start 166.624 98.922) (end 166.624 97.282) (width 0.5) (layer "F.Cu") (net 5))
 (segment (start 148.844 101.512) (end 148.604 101.752) (width 0.5) (layer "B.Cu") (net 5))
 (segment (start 148.844 98.922) (end 148.844 101.512) (width 0.5) (layer "B.Cu") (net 5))
 (segment (start 166.624 98.922) (end 166.624 101.752) (width 0.5) (layer "B.Cu") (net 5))
 (segment (start 148.604 101.752) (end 148.604 102.006) (width 0.5) (layer "B.Cu") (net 5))
 (segment (start 166.624 101.752) (end 166.384 101.992) (width 0.5) (layer "B.Cu") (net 5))
 (segment (start 171.704 94.742) (end 169.164 94.742) (width 0.5) (layer "B.Cu") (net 52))
 (segment (start 169.404 101.752) (end 169.404 99.162) (width 0.5) (layer "B.Cu") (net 52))
 (segment (start 169.404 99.162) (end 169.164 98.922) (width 0.5) (layer "B.Cu") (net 52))
 (segment (start 169.164 94.742) (end 169.164 98.922) (width 0.5) (layer "B.Cu") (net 52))
 (segment (start 169.15 102.006) (end 169.404 101.752) (width 0.5) (layer "B.Cu") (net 52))
 (segment (start 157.226 92.71) (end 156.21 93.726) (width 0.5) (layer "F.Cu") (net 3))
 (segment (start 173.228 92.71) (end 157.226 92.71) (width 0.5) (layer "F.Cu") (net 3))
 (segment (start 174.244 94.742) (end 174.244 93.218) (width 0.5) (layer "F.Cu") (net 3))
 (segment (start 156.21 93.726) (end 156.21 94.742) (width 0.5) (layer "F.Cu") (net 3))
 (segment (start 174.244 93.218) (end 173.228 92.71) (width 0.5) (layer "F.Cu") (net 3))
 (segment (start 171.704 98.922) (end 173.366 98.922) (width 0.5) (layer "B.Cu") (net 3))
 (segment (start 174.244 98.044) (end 174.244 94.742) (width 0.5) (layer "B.Cu") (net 3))
 (segment (start 156.21 94.742) (end 153.924 97.028) (width 0.5) (layer "B.Cu") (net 3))
 (segment (start 171.45 102.006) (end 171.704 101.752) (width 0.5) (layer "B.Cu") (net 3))
 (segment (start 173.366 98.922) (end 174.244 98.044) (width 0.5) (layer "B.Cu") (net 3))
 (segment (start 153.924 102.006) (end 153.924 108.306) (width 0.5) (layer "B.Cu") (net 3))
 (segment (start 171.45 102.006) (end 171.45 108.306) (width 0.5) (layer "B.Cu") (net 3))
 (segment (start 153.924 98.552) (end 153.924 102.006) (width 0.5) (layer "B.Cu") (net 3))
 (segment (start 171.704 101.752) (end 171.704 98.922) (width 0.5) (layer "B.Cu") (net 3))
 (segment (start 153.924 97.028) (end 153.924 98.552) (width 0.5) (layer "B.Cu") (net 3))
 (segment (start 177.698 101.752) (end 178.308 102.362) (width 0.5) (layer "B.Cu") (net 55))
 (segment (start 174.258 102.006) (end 173.75 102.006) (width 0.5) (layer "B.Cu") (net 55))
 (segment (start 174.614 102.362) (end 174.258 102.006) (width 0.5) (layer "B.Cu") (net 55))
 (segment (start 177.8 102.362) (end 174.614 102.362) (width 0.5) (layer "B.Cu") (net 55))
 (segment (start 164.084 101.992) (end 164.084 97.282) (width 0.2) (layer "B.Cu") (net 53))
 (segment (start 164.084 108.292) (end 164.084 101.992) (width 0.5) (layer "B.Cu") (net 53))
 (segment (start 164.084 97.282) (end 161.544 94.742) (width 0.2) (layer "B.Cu") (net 53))
 (segment (start 151.384 97.028) (end 151.638 96.774) (width 0.5) (layer "B.Cu") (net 4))
 (segment (start 151.384 101.512) (end 151.624 101.752) (width 0.5) (layer "B.Cu") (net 4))
 (segment (start 151.624 102.006) (end 151.624 100.852) (width 0.5) (layer "B.Cu") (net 4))
 (segment (start 151.384 97.028) (end 151.384 98.552) (width 0.5) (layer "B.Cu") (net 4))
 (segment (start 151.638 96.774) (end 151.638 94.742) (width 0.5) (layer "B.Cu") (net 4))
 (segment (start 151.638 94.742) (end 153.67 94.742) (width 0.5) (layer "B.Cu") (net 4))
 (segment (start 151.624 101.752) (end 151.624 102.006) (width 0.5) (layer "B.Cu") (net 4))
 (segment (start 151.384 98.552) (end 151.384 101.512) (width 0.5) (layer "B.Cu") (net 4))
 (segment (start 177.8 104.902) (end 177.546 105.156) (width 0.5) (layer "F.Cu") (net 54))
 (segment (start 156.21 105.156) (end 156.21 101.6) (width 0.5) (layer "F.Cu") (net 54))
 (segment (start 177.546 105.156) (end 156.21 105.156) (width 0.5) (layer "F.Cu") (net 54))
 (segment (start 146.304 102.006) (end 146.304 108.306) (width 0.5) (layer "B.Cu") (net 56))
 (segment (start 146.304 96.52) (end 146.304 102.006) (width 0.5) (layer "B.Cu") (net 56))
 (segment (start 144.526 94.742) (end 146.304 96.52) (width 0.5) (layer "B.Cu") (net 56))
 (segment (start 144.018 94.742) (end 144.526 94.742) (width 0.5) (layer "B.Cu") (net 56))
 (segment (start 140.462 102.224) (end 140.462 102.362) (width 0.5) (layer "F.Cu") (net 48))
 (segment (start 143.764 101.512) (end 144.004 101.752) (width 0.5) (layer "B.Cu") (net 48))
 (segment (start 143.394 102.362) (end 143.75 102.006) (width 0.5) (layer "B.Cu") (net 48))
 (segment (start 140.462 102.362) (end 143.394 102.362) (width 0.5) (layer "B.Cu") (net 48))
 (segment (start 144.004 101.752) (end 144.004 102.006) (width 0.5) (layer "B.Cu") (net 48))
 (segment (start 143.764 98.922) (end 143.764 101.512) (width 0.5) (layer "B.Cu") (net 48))
 (segment (start 143.75 102.006) (end 144.004 102.006) (width 0.5) (layer "B.Cu") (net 48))
 (segment (start 161.784 101.992) (end 161.174 101.992) (width 0.2) (layer "B.Cu") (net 8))
 (segment (start 161.544 98.922) (end 161.544 101.752) (width 0.5) (layer "B.Cu") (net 8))
 (segment (start 161.174 101.992) (end 158.496 99.314) (width 0.2) (layer "B.Cu") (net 8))
 (segment (start 161.544 101.752) (end 161.784 101.992) (width 0.5) (layer "B.Cu") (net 8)))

